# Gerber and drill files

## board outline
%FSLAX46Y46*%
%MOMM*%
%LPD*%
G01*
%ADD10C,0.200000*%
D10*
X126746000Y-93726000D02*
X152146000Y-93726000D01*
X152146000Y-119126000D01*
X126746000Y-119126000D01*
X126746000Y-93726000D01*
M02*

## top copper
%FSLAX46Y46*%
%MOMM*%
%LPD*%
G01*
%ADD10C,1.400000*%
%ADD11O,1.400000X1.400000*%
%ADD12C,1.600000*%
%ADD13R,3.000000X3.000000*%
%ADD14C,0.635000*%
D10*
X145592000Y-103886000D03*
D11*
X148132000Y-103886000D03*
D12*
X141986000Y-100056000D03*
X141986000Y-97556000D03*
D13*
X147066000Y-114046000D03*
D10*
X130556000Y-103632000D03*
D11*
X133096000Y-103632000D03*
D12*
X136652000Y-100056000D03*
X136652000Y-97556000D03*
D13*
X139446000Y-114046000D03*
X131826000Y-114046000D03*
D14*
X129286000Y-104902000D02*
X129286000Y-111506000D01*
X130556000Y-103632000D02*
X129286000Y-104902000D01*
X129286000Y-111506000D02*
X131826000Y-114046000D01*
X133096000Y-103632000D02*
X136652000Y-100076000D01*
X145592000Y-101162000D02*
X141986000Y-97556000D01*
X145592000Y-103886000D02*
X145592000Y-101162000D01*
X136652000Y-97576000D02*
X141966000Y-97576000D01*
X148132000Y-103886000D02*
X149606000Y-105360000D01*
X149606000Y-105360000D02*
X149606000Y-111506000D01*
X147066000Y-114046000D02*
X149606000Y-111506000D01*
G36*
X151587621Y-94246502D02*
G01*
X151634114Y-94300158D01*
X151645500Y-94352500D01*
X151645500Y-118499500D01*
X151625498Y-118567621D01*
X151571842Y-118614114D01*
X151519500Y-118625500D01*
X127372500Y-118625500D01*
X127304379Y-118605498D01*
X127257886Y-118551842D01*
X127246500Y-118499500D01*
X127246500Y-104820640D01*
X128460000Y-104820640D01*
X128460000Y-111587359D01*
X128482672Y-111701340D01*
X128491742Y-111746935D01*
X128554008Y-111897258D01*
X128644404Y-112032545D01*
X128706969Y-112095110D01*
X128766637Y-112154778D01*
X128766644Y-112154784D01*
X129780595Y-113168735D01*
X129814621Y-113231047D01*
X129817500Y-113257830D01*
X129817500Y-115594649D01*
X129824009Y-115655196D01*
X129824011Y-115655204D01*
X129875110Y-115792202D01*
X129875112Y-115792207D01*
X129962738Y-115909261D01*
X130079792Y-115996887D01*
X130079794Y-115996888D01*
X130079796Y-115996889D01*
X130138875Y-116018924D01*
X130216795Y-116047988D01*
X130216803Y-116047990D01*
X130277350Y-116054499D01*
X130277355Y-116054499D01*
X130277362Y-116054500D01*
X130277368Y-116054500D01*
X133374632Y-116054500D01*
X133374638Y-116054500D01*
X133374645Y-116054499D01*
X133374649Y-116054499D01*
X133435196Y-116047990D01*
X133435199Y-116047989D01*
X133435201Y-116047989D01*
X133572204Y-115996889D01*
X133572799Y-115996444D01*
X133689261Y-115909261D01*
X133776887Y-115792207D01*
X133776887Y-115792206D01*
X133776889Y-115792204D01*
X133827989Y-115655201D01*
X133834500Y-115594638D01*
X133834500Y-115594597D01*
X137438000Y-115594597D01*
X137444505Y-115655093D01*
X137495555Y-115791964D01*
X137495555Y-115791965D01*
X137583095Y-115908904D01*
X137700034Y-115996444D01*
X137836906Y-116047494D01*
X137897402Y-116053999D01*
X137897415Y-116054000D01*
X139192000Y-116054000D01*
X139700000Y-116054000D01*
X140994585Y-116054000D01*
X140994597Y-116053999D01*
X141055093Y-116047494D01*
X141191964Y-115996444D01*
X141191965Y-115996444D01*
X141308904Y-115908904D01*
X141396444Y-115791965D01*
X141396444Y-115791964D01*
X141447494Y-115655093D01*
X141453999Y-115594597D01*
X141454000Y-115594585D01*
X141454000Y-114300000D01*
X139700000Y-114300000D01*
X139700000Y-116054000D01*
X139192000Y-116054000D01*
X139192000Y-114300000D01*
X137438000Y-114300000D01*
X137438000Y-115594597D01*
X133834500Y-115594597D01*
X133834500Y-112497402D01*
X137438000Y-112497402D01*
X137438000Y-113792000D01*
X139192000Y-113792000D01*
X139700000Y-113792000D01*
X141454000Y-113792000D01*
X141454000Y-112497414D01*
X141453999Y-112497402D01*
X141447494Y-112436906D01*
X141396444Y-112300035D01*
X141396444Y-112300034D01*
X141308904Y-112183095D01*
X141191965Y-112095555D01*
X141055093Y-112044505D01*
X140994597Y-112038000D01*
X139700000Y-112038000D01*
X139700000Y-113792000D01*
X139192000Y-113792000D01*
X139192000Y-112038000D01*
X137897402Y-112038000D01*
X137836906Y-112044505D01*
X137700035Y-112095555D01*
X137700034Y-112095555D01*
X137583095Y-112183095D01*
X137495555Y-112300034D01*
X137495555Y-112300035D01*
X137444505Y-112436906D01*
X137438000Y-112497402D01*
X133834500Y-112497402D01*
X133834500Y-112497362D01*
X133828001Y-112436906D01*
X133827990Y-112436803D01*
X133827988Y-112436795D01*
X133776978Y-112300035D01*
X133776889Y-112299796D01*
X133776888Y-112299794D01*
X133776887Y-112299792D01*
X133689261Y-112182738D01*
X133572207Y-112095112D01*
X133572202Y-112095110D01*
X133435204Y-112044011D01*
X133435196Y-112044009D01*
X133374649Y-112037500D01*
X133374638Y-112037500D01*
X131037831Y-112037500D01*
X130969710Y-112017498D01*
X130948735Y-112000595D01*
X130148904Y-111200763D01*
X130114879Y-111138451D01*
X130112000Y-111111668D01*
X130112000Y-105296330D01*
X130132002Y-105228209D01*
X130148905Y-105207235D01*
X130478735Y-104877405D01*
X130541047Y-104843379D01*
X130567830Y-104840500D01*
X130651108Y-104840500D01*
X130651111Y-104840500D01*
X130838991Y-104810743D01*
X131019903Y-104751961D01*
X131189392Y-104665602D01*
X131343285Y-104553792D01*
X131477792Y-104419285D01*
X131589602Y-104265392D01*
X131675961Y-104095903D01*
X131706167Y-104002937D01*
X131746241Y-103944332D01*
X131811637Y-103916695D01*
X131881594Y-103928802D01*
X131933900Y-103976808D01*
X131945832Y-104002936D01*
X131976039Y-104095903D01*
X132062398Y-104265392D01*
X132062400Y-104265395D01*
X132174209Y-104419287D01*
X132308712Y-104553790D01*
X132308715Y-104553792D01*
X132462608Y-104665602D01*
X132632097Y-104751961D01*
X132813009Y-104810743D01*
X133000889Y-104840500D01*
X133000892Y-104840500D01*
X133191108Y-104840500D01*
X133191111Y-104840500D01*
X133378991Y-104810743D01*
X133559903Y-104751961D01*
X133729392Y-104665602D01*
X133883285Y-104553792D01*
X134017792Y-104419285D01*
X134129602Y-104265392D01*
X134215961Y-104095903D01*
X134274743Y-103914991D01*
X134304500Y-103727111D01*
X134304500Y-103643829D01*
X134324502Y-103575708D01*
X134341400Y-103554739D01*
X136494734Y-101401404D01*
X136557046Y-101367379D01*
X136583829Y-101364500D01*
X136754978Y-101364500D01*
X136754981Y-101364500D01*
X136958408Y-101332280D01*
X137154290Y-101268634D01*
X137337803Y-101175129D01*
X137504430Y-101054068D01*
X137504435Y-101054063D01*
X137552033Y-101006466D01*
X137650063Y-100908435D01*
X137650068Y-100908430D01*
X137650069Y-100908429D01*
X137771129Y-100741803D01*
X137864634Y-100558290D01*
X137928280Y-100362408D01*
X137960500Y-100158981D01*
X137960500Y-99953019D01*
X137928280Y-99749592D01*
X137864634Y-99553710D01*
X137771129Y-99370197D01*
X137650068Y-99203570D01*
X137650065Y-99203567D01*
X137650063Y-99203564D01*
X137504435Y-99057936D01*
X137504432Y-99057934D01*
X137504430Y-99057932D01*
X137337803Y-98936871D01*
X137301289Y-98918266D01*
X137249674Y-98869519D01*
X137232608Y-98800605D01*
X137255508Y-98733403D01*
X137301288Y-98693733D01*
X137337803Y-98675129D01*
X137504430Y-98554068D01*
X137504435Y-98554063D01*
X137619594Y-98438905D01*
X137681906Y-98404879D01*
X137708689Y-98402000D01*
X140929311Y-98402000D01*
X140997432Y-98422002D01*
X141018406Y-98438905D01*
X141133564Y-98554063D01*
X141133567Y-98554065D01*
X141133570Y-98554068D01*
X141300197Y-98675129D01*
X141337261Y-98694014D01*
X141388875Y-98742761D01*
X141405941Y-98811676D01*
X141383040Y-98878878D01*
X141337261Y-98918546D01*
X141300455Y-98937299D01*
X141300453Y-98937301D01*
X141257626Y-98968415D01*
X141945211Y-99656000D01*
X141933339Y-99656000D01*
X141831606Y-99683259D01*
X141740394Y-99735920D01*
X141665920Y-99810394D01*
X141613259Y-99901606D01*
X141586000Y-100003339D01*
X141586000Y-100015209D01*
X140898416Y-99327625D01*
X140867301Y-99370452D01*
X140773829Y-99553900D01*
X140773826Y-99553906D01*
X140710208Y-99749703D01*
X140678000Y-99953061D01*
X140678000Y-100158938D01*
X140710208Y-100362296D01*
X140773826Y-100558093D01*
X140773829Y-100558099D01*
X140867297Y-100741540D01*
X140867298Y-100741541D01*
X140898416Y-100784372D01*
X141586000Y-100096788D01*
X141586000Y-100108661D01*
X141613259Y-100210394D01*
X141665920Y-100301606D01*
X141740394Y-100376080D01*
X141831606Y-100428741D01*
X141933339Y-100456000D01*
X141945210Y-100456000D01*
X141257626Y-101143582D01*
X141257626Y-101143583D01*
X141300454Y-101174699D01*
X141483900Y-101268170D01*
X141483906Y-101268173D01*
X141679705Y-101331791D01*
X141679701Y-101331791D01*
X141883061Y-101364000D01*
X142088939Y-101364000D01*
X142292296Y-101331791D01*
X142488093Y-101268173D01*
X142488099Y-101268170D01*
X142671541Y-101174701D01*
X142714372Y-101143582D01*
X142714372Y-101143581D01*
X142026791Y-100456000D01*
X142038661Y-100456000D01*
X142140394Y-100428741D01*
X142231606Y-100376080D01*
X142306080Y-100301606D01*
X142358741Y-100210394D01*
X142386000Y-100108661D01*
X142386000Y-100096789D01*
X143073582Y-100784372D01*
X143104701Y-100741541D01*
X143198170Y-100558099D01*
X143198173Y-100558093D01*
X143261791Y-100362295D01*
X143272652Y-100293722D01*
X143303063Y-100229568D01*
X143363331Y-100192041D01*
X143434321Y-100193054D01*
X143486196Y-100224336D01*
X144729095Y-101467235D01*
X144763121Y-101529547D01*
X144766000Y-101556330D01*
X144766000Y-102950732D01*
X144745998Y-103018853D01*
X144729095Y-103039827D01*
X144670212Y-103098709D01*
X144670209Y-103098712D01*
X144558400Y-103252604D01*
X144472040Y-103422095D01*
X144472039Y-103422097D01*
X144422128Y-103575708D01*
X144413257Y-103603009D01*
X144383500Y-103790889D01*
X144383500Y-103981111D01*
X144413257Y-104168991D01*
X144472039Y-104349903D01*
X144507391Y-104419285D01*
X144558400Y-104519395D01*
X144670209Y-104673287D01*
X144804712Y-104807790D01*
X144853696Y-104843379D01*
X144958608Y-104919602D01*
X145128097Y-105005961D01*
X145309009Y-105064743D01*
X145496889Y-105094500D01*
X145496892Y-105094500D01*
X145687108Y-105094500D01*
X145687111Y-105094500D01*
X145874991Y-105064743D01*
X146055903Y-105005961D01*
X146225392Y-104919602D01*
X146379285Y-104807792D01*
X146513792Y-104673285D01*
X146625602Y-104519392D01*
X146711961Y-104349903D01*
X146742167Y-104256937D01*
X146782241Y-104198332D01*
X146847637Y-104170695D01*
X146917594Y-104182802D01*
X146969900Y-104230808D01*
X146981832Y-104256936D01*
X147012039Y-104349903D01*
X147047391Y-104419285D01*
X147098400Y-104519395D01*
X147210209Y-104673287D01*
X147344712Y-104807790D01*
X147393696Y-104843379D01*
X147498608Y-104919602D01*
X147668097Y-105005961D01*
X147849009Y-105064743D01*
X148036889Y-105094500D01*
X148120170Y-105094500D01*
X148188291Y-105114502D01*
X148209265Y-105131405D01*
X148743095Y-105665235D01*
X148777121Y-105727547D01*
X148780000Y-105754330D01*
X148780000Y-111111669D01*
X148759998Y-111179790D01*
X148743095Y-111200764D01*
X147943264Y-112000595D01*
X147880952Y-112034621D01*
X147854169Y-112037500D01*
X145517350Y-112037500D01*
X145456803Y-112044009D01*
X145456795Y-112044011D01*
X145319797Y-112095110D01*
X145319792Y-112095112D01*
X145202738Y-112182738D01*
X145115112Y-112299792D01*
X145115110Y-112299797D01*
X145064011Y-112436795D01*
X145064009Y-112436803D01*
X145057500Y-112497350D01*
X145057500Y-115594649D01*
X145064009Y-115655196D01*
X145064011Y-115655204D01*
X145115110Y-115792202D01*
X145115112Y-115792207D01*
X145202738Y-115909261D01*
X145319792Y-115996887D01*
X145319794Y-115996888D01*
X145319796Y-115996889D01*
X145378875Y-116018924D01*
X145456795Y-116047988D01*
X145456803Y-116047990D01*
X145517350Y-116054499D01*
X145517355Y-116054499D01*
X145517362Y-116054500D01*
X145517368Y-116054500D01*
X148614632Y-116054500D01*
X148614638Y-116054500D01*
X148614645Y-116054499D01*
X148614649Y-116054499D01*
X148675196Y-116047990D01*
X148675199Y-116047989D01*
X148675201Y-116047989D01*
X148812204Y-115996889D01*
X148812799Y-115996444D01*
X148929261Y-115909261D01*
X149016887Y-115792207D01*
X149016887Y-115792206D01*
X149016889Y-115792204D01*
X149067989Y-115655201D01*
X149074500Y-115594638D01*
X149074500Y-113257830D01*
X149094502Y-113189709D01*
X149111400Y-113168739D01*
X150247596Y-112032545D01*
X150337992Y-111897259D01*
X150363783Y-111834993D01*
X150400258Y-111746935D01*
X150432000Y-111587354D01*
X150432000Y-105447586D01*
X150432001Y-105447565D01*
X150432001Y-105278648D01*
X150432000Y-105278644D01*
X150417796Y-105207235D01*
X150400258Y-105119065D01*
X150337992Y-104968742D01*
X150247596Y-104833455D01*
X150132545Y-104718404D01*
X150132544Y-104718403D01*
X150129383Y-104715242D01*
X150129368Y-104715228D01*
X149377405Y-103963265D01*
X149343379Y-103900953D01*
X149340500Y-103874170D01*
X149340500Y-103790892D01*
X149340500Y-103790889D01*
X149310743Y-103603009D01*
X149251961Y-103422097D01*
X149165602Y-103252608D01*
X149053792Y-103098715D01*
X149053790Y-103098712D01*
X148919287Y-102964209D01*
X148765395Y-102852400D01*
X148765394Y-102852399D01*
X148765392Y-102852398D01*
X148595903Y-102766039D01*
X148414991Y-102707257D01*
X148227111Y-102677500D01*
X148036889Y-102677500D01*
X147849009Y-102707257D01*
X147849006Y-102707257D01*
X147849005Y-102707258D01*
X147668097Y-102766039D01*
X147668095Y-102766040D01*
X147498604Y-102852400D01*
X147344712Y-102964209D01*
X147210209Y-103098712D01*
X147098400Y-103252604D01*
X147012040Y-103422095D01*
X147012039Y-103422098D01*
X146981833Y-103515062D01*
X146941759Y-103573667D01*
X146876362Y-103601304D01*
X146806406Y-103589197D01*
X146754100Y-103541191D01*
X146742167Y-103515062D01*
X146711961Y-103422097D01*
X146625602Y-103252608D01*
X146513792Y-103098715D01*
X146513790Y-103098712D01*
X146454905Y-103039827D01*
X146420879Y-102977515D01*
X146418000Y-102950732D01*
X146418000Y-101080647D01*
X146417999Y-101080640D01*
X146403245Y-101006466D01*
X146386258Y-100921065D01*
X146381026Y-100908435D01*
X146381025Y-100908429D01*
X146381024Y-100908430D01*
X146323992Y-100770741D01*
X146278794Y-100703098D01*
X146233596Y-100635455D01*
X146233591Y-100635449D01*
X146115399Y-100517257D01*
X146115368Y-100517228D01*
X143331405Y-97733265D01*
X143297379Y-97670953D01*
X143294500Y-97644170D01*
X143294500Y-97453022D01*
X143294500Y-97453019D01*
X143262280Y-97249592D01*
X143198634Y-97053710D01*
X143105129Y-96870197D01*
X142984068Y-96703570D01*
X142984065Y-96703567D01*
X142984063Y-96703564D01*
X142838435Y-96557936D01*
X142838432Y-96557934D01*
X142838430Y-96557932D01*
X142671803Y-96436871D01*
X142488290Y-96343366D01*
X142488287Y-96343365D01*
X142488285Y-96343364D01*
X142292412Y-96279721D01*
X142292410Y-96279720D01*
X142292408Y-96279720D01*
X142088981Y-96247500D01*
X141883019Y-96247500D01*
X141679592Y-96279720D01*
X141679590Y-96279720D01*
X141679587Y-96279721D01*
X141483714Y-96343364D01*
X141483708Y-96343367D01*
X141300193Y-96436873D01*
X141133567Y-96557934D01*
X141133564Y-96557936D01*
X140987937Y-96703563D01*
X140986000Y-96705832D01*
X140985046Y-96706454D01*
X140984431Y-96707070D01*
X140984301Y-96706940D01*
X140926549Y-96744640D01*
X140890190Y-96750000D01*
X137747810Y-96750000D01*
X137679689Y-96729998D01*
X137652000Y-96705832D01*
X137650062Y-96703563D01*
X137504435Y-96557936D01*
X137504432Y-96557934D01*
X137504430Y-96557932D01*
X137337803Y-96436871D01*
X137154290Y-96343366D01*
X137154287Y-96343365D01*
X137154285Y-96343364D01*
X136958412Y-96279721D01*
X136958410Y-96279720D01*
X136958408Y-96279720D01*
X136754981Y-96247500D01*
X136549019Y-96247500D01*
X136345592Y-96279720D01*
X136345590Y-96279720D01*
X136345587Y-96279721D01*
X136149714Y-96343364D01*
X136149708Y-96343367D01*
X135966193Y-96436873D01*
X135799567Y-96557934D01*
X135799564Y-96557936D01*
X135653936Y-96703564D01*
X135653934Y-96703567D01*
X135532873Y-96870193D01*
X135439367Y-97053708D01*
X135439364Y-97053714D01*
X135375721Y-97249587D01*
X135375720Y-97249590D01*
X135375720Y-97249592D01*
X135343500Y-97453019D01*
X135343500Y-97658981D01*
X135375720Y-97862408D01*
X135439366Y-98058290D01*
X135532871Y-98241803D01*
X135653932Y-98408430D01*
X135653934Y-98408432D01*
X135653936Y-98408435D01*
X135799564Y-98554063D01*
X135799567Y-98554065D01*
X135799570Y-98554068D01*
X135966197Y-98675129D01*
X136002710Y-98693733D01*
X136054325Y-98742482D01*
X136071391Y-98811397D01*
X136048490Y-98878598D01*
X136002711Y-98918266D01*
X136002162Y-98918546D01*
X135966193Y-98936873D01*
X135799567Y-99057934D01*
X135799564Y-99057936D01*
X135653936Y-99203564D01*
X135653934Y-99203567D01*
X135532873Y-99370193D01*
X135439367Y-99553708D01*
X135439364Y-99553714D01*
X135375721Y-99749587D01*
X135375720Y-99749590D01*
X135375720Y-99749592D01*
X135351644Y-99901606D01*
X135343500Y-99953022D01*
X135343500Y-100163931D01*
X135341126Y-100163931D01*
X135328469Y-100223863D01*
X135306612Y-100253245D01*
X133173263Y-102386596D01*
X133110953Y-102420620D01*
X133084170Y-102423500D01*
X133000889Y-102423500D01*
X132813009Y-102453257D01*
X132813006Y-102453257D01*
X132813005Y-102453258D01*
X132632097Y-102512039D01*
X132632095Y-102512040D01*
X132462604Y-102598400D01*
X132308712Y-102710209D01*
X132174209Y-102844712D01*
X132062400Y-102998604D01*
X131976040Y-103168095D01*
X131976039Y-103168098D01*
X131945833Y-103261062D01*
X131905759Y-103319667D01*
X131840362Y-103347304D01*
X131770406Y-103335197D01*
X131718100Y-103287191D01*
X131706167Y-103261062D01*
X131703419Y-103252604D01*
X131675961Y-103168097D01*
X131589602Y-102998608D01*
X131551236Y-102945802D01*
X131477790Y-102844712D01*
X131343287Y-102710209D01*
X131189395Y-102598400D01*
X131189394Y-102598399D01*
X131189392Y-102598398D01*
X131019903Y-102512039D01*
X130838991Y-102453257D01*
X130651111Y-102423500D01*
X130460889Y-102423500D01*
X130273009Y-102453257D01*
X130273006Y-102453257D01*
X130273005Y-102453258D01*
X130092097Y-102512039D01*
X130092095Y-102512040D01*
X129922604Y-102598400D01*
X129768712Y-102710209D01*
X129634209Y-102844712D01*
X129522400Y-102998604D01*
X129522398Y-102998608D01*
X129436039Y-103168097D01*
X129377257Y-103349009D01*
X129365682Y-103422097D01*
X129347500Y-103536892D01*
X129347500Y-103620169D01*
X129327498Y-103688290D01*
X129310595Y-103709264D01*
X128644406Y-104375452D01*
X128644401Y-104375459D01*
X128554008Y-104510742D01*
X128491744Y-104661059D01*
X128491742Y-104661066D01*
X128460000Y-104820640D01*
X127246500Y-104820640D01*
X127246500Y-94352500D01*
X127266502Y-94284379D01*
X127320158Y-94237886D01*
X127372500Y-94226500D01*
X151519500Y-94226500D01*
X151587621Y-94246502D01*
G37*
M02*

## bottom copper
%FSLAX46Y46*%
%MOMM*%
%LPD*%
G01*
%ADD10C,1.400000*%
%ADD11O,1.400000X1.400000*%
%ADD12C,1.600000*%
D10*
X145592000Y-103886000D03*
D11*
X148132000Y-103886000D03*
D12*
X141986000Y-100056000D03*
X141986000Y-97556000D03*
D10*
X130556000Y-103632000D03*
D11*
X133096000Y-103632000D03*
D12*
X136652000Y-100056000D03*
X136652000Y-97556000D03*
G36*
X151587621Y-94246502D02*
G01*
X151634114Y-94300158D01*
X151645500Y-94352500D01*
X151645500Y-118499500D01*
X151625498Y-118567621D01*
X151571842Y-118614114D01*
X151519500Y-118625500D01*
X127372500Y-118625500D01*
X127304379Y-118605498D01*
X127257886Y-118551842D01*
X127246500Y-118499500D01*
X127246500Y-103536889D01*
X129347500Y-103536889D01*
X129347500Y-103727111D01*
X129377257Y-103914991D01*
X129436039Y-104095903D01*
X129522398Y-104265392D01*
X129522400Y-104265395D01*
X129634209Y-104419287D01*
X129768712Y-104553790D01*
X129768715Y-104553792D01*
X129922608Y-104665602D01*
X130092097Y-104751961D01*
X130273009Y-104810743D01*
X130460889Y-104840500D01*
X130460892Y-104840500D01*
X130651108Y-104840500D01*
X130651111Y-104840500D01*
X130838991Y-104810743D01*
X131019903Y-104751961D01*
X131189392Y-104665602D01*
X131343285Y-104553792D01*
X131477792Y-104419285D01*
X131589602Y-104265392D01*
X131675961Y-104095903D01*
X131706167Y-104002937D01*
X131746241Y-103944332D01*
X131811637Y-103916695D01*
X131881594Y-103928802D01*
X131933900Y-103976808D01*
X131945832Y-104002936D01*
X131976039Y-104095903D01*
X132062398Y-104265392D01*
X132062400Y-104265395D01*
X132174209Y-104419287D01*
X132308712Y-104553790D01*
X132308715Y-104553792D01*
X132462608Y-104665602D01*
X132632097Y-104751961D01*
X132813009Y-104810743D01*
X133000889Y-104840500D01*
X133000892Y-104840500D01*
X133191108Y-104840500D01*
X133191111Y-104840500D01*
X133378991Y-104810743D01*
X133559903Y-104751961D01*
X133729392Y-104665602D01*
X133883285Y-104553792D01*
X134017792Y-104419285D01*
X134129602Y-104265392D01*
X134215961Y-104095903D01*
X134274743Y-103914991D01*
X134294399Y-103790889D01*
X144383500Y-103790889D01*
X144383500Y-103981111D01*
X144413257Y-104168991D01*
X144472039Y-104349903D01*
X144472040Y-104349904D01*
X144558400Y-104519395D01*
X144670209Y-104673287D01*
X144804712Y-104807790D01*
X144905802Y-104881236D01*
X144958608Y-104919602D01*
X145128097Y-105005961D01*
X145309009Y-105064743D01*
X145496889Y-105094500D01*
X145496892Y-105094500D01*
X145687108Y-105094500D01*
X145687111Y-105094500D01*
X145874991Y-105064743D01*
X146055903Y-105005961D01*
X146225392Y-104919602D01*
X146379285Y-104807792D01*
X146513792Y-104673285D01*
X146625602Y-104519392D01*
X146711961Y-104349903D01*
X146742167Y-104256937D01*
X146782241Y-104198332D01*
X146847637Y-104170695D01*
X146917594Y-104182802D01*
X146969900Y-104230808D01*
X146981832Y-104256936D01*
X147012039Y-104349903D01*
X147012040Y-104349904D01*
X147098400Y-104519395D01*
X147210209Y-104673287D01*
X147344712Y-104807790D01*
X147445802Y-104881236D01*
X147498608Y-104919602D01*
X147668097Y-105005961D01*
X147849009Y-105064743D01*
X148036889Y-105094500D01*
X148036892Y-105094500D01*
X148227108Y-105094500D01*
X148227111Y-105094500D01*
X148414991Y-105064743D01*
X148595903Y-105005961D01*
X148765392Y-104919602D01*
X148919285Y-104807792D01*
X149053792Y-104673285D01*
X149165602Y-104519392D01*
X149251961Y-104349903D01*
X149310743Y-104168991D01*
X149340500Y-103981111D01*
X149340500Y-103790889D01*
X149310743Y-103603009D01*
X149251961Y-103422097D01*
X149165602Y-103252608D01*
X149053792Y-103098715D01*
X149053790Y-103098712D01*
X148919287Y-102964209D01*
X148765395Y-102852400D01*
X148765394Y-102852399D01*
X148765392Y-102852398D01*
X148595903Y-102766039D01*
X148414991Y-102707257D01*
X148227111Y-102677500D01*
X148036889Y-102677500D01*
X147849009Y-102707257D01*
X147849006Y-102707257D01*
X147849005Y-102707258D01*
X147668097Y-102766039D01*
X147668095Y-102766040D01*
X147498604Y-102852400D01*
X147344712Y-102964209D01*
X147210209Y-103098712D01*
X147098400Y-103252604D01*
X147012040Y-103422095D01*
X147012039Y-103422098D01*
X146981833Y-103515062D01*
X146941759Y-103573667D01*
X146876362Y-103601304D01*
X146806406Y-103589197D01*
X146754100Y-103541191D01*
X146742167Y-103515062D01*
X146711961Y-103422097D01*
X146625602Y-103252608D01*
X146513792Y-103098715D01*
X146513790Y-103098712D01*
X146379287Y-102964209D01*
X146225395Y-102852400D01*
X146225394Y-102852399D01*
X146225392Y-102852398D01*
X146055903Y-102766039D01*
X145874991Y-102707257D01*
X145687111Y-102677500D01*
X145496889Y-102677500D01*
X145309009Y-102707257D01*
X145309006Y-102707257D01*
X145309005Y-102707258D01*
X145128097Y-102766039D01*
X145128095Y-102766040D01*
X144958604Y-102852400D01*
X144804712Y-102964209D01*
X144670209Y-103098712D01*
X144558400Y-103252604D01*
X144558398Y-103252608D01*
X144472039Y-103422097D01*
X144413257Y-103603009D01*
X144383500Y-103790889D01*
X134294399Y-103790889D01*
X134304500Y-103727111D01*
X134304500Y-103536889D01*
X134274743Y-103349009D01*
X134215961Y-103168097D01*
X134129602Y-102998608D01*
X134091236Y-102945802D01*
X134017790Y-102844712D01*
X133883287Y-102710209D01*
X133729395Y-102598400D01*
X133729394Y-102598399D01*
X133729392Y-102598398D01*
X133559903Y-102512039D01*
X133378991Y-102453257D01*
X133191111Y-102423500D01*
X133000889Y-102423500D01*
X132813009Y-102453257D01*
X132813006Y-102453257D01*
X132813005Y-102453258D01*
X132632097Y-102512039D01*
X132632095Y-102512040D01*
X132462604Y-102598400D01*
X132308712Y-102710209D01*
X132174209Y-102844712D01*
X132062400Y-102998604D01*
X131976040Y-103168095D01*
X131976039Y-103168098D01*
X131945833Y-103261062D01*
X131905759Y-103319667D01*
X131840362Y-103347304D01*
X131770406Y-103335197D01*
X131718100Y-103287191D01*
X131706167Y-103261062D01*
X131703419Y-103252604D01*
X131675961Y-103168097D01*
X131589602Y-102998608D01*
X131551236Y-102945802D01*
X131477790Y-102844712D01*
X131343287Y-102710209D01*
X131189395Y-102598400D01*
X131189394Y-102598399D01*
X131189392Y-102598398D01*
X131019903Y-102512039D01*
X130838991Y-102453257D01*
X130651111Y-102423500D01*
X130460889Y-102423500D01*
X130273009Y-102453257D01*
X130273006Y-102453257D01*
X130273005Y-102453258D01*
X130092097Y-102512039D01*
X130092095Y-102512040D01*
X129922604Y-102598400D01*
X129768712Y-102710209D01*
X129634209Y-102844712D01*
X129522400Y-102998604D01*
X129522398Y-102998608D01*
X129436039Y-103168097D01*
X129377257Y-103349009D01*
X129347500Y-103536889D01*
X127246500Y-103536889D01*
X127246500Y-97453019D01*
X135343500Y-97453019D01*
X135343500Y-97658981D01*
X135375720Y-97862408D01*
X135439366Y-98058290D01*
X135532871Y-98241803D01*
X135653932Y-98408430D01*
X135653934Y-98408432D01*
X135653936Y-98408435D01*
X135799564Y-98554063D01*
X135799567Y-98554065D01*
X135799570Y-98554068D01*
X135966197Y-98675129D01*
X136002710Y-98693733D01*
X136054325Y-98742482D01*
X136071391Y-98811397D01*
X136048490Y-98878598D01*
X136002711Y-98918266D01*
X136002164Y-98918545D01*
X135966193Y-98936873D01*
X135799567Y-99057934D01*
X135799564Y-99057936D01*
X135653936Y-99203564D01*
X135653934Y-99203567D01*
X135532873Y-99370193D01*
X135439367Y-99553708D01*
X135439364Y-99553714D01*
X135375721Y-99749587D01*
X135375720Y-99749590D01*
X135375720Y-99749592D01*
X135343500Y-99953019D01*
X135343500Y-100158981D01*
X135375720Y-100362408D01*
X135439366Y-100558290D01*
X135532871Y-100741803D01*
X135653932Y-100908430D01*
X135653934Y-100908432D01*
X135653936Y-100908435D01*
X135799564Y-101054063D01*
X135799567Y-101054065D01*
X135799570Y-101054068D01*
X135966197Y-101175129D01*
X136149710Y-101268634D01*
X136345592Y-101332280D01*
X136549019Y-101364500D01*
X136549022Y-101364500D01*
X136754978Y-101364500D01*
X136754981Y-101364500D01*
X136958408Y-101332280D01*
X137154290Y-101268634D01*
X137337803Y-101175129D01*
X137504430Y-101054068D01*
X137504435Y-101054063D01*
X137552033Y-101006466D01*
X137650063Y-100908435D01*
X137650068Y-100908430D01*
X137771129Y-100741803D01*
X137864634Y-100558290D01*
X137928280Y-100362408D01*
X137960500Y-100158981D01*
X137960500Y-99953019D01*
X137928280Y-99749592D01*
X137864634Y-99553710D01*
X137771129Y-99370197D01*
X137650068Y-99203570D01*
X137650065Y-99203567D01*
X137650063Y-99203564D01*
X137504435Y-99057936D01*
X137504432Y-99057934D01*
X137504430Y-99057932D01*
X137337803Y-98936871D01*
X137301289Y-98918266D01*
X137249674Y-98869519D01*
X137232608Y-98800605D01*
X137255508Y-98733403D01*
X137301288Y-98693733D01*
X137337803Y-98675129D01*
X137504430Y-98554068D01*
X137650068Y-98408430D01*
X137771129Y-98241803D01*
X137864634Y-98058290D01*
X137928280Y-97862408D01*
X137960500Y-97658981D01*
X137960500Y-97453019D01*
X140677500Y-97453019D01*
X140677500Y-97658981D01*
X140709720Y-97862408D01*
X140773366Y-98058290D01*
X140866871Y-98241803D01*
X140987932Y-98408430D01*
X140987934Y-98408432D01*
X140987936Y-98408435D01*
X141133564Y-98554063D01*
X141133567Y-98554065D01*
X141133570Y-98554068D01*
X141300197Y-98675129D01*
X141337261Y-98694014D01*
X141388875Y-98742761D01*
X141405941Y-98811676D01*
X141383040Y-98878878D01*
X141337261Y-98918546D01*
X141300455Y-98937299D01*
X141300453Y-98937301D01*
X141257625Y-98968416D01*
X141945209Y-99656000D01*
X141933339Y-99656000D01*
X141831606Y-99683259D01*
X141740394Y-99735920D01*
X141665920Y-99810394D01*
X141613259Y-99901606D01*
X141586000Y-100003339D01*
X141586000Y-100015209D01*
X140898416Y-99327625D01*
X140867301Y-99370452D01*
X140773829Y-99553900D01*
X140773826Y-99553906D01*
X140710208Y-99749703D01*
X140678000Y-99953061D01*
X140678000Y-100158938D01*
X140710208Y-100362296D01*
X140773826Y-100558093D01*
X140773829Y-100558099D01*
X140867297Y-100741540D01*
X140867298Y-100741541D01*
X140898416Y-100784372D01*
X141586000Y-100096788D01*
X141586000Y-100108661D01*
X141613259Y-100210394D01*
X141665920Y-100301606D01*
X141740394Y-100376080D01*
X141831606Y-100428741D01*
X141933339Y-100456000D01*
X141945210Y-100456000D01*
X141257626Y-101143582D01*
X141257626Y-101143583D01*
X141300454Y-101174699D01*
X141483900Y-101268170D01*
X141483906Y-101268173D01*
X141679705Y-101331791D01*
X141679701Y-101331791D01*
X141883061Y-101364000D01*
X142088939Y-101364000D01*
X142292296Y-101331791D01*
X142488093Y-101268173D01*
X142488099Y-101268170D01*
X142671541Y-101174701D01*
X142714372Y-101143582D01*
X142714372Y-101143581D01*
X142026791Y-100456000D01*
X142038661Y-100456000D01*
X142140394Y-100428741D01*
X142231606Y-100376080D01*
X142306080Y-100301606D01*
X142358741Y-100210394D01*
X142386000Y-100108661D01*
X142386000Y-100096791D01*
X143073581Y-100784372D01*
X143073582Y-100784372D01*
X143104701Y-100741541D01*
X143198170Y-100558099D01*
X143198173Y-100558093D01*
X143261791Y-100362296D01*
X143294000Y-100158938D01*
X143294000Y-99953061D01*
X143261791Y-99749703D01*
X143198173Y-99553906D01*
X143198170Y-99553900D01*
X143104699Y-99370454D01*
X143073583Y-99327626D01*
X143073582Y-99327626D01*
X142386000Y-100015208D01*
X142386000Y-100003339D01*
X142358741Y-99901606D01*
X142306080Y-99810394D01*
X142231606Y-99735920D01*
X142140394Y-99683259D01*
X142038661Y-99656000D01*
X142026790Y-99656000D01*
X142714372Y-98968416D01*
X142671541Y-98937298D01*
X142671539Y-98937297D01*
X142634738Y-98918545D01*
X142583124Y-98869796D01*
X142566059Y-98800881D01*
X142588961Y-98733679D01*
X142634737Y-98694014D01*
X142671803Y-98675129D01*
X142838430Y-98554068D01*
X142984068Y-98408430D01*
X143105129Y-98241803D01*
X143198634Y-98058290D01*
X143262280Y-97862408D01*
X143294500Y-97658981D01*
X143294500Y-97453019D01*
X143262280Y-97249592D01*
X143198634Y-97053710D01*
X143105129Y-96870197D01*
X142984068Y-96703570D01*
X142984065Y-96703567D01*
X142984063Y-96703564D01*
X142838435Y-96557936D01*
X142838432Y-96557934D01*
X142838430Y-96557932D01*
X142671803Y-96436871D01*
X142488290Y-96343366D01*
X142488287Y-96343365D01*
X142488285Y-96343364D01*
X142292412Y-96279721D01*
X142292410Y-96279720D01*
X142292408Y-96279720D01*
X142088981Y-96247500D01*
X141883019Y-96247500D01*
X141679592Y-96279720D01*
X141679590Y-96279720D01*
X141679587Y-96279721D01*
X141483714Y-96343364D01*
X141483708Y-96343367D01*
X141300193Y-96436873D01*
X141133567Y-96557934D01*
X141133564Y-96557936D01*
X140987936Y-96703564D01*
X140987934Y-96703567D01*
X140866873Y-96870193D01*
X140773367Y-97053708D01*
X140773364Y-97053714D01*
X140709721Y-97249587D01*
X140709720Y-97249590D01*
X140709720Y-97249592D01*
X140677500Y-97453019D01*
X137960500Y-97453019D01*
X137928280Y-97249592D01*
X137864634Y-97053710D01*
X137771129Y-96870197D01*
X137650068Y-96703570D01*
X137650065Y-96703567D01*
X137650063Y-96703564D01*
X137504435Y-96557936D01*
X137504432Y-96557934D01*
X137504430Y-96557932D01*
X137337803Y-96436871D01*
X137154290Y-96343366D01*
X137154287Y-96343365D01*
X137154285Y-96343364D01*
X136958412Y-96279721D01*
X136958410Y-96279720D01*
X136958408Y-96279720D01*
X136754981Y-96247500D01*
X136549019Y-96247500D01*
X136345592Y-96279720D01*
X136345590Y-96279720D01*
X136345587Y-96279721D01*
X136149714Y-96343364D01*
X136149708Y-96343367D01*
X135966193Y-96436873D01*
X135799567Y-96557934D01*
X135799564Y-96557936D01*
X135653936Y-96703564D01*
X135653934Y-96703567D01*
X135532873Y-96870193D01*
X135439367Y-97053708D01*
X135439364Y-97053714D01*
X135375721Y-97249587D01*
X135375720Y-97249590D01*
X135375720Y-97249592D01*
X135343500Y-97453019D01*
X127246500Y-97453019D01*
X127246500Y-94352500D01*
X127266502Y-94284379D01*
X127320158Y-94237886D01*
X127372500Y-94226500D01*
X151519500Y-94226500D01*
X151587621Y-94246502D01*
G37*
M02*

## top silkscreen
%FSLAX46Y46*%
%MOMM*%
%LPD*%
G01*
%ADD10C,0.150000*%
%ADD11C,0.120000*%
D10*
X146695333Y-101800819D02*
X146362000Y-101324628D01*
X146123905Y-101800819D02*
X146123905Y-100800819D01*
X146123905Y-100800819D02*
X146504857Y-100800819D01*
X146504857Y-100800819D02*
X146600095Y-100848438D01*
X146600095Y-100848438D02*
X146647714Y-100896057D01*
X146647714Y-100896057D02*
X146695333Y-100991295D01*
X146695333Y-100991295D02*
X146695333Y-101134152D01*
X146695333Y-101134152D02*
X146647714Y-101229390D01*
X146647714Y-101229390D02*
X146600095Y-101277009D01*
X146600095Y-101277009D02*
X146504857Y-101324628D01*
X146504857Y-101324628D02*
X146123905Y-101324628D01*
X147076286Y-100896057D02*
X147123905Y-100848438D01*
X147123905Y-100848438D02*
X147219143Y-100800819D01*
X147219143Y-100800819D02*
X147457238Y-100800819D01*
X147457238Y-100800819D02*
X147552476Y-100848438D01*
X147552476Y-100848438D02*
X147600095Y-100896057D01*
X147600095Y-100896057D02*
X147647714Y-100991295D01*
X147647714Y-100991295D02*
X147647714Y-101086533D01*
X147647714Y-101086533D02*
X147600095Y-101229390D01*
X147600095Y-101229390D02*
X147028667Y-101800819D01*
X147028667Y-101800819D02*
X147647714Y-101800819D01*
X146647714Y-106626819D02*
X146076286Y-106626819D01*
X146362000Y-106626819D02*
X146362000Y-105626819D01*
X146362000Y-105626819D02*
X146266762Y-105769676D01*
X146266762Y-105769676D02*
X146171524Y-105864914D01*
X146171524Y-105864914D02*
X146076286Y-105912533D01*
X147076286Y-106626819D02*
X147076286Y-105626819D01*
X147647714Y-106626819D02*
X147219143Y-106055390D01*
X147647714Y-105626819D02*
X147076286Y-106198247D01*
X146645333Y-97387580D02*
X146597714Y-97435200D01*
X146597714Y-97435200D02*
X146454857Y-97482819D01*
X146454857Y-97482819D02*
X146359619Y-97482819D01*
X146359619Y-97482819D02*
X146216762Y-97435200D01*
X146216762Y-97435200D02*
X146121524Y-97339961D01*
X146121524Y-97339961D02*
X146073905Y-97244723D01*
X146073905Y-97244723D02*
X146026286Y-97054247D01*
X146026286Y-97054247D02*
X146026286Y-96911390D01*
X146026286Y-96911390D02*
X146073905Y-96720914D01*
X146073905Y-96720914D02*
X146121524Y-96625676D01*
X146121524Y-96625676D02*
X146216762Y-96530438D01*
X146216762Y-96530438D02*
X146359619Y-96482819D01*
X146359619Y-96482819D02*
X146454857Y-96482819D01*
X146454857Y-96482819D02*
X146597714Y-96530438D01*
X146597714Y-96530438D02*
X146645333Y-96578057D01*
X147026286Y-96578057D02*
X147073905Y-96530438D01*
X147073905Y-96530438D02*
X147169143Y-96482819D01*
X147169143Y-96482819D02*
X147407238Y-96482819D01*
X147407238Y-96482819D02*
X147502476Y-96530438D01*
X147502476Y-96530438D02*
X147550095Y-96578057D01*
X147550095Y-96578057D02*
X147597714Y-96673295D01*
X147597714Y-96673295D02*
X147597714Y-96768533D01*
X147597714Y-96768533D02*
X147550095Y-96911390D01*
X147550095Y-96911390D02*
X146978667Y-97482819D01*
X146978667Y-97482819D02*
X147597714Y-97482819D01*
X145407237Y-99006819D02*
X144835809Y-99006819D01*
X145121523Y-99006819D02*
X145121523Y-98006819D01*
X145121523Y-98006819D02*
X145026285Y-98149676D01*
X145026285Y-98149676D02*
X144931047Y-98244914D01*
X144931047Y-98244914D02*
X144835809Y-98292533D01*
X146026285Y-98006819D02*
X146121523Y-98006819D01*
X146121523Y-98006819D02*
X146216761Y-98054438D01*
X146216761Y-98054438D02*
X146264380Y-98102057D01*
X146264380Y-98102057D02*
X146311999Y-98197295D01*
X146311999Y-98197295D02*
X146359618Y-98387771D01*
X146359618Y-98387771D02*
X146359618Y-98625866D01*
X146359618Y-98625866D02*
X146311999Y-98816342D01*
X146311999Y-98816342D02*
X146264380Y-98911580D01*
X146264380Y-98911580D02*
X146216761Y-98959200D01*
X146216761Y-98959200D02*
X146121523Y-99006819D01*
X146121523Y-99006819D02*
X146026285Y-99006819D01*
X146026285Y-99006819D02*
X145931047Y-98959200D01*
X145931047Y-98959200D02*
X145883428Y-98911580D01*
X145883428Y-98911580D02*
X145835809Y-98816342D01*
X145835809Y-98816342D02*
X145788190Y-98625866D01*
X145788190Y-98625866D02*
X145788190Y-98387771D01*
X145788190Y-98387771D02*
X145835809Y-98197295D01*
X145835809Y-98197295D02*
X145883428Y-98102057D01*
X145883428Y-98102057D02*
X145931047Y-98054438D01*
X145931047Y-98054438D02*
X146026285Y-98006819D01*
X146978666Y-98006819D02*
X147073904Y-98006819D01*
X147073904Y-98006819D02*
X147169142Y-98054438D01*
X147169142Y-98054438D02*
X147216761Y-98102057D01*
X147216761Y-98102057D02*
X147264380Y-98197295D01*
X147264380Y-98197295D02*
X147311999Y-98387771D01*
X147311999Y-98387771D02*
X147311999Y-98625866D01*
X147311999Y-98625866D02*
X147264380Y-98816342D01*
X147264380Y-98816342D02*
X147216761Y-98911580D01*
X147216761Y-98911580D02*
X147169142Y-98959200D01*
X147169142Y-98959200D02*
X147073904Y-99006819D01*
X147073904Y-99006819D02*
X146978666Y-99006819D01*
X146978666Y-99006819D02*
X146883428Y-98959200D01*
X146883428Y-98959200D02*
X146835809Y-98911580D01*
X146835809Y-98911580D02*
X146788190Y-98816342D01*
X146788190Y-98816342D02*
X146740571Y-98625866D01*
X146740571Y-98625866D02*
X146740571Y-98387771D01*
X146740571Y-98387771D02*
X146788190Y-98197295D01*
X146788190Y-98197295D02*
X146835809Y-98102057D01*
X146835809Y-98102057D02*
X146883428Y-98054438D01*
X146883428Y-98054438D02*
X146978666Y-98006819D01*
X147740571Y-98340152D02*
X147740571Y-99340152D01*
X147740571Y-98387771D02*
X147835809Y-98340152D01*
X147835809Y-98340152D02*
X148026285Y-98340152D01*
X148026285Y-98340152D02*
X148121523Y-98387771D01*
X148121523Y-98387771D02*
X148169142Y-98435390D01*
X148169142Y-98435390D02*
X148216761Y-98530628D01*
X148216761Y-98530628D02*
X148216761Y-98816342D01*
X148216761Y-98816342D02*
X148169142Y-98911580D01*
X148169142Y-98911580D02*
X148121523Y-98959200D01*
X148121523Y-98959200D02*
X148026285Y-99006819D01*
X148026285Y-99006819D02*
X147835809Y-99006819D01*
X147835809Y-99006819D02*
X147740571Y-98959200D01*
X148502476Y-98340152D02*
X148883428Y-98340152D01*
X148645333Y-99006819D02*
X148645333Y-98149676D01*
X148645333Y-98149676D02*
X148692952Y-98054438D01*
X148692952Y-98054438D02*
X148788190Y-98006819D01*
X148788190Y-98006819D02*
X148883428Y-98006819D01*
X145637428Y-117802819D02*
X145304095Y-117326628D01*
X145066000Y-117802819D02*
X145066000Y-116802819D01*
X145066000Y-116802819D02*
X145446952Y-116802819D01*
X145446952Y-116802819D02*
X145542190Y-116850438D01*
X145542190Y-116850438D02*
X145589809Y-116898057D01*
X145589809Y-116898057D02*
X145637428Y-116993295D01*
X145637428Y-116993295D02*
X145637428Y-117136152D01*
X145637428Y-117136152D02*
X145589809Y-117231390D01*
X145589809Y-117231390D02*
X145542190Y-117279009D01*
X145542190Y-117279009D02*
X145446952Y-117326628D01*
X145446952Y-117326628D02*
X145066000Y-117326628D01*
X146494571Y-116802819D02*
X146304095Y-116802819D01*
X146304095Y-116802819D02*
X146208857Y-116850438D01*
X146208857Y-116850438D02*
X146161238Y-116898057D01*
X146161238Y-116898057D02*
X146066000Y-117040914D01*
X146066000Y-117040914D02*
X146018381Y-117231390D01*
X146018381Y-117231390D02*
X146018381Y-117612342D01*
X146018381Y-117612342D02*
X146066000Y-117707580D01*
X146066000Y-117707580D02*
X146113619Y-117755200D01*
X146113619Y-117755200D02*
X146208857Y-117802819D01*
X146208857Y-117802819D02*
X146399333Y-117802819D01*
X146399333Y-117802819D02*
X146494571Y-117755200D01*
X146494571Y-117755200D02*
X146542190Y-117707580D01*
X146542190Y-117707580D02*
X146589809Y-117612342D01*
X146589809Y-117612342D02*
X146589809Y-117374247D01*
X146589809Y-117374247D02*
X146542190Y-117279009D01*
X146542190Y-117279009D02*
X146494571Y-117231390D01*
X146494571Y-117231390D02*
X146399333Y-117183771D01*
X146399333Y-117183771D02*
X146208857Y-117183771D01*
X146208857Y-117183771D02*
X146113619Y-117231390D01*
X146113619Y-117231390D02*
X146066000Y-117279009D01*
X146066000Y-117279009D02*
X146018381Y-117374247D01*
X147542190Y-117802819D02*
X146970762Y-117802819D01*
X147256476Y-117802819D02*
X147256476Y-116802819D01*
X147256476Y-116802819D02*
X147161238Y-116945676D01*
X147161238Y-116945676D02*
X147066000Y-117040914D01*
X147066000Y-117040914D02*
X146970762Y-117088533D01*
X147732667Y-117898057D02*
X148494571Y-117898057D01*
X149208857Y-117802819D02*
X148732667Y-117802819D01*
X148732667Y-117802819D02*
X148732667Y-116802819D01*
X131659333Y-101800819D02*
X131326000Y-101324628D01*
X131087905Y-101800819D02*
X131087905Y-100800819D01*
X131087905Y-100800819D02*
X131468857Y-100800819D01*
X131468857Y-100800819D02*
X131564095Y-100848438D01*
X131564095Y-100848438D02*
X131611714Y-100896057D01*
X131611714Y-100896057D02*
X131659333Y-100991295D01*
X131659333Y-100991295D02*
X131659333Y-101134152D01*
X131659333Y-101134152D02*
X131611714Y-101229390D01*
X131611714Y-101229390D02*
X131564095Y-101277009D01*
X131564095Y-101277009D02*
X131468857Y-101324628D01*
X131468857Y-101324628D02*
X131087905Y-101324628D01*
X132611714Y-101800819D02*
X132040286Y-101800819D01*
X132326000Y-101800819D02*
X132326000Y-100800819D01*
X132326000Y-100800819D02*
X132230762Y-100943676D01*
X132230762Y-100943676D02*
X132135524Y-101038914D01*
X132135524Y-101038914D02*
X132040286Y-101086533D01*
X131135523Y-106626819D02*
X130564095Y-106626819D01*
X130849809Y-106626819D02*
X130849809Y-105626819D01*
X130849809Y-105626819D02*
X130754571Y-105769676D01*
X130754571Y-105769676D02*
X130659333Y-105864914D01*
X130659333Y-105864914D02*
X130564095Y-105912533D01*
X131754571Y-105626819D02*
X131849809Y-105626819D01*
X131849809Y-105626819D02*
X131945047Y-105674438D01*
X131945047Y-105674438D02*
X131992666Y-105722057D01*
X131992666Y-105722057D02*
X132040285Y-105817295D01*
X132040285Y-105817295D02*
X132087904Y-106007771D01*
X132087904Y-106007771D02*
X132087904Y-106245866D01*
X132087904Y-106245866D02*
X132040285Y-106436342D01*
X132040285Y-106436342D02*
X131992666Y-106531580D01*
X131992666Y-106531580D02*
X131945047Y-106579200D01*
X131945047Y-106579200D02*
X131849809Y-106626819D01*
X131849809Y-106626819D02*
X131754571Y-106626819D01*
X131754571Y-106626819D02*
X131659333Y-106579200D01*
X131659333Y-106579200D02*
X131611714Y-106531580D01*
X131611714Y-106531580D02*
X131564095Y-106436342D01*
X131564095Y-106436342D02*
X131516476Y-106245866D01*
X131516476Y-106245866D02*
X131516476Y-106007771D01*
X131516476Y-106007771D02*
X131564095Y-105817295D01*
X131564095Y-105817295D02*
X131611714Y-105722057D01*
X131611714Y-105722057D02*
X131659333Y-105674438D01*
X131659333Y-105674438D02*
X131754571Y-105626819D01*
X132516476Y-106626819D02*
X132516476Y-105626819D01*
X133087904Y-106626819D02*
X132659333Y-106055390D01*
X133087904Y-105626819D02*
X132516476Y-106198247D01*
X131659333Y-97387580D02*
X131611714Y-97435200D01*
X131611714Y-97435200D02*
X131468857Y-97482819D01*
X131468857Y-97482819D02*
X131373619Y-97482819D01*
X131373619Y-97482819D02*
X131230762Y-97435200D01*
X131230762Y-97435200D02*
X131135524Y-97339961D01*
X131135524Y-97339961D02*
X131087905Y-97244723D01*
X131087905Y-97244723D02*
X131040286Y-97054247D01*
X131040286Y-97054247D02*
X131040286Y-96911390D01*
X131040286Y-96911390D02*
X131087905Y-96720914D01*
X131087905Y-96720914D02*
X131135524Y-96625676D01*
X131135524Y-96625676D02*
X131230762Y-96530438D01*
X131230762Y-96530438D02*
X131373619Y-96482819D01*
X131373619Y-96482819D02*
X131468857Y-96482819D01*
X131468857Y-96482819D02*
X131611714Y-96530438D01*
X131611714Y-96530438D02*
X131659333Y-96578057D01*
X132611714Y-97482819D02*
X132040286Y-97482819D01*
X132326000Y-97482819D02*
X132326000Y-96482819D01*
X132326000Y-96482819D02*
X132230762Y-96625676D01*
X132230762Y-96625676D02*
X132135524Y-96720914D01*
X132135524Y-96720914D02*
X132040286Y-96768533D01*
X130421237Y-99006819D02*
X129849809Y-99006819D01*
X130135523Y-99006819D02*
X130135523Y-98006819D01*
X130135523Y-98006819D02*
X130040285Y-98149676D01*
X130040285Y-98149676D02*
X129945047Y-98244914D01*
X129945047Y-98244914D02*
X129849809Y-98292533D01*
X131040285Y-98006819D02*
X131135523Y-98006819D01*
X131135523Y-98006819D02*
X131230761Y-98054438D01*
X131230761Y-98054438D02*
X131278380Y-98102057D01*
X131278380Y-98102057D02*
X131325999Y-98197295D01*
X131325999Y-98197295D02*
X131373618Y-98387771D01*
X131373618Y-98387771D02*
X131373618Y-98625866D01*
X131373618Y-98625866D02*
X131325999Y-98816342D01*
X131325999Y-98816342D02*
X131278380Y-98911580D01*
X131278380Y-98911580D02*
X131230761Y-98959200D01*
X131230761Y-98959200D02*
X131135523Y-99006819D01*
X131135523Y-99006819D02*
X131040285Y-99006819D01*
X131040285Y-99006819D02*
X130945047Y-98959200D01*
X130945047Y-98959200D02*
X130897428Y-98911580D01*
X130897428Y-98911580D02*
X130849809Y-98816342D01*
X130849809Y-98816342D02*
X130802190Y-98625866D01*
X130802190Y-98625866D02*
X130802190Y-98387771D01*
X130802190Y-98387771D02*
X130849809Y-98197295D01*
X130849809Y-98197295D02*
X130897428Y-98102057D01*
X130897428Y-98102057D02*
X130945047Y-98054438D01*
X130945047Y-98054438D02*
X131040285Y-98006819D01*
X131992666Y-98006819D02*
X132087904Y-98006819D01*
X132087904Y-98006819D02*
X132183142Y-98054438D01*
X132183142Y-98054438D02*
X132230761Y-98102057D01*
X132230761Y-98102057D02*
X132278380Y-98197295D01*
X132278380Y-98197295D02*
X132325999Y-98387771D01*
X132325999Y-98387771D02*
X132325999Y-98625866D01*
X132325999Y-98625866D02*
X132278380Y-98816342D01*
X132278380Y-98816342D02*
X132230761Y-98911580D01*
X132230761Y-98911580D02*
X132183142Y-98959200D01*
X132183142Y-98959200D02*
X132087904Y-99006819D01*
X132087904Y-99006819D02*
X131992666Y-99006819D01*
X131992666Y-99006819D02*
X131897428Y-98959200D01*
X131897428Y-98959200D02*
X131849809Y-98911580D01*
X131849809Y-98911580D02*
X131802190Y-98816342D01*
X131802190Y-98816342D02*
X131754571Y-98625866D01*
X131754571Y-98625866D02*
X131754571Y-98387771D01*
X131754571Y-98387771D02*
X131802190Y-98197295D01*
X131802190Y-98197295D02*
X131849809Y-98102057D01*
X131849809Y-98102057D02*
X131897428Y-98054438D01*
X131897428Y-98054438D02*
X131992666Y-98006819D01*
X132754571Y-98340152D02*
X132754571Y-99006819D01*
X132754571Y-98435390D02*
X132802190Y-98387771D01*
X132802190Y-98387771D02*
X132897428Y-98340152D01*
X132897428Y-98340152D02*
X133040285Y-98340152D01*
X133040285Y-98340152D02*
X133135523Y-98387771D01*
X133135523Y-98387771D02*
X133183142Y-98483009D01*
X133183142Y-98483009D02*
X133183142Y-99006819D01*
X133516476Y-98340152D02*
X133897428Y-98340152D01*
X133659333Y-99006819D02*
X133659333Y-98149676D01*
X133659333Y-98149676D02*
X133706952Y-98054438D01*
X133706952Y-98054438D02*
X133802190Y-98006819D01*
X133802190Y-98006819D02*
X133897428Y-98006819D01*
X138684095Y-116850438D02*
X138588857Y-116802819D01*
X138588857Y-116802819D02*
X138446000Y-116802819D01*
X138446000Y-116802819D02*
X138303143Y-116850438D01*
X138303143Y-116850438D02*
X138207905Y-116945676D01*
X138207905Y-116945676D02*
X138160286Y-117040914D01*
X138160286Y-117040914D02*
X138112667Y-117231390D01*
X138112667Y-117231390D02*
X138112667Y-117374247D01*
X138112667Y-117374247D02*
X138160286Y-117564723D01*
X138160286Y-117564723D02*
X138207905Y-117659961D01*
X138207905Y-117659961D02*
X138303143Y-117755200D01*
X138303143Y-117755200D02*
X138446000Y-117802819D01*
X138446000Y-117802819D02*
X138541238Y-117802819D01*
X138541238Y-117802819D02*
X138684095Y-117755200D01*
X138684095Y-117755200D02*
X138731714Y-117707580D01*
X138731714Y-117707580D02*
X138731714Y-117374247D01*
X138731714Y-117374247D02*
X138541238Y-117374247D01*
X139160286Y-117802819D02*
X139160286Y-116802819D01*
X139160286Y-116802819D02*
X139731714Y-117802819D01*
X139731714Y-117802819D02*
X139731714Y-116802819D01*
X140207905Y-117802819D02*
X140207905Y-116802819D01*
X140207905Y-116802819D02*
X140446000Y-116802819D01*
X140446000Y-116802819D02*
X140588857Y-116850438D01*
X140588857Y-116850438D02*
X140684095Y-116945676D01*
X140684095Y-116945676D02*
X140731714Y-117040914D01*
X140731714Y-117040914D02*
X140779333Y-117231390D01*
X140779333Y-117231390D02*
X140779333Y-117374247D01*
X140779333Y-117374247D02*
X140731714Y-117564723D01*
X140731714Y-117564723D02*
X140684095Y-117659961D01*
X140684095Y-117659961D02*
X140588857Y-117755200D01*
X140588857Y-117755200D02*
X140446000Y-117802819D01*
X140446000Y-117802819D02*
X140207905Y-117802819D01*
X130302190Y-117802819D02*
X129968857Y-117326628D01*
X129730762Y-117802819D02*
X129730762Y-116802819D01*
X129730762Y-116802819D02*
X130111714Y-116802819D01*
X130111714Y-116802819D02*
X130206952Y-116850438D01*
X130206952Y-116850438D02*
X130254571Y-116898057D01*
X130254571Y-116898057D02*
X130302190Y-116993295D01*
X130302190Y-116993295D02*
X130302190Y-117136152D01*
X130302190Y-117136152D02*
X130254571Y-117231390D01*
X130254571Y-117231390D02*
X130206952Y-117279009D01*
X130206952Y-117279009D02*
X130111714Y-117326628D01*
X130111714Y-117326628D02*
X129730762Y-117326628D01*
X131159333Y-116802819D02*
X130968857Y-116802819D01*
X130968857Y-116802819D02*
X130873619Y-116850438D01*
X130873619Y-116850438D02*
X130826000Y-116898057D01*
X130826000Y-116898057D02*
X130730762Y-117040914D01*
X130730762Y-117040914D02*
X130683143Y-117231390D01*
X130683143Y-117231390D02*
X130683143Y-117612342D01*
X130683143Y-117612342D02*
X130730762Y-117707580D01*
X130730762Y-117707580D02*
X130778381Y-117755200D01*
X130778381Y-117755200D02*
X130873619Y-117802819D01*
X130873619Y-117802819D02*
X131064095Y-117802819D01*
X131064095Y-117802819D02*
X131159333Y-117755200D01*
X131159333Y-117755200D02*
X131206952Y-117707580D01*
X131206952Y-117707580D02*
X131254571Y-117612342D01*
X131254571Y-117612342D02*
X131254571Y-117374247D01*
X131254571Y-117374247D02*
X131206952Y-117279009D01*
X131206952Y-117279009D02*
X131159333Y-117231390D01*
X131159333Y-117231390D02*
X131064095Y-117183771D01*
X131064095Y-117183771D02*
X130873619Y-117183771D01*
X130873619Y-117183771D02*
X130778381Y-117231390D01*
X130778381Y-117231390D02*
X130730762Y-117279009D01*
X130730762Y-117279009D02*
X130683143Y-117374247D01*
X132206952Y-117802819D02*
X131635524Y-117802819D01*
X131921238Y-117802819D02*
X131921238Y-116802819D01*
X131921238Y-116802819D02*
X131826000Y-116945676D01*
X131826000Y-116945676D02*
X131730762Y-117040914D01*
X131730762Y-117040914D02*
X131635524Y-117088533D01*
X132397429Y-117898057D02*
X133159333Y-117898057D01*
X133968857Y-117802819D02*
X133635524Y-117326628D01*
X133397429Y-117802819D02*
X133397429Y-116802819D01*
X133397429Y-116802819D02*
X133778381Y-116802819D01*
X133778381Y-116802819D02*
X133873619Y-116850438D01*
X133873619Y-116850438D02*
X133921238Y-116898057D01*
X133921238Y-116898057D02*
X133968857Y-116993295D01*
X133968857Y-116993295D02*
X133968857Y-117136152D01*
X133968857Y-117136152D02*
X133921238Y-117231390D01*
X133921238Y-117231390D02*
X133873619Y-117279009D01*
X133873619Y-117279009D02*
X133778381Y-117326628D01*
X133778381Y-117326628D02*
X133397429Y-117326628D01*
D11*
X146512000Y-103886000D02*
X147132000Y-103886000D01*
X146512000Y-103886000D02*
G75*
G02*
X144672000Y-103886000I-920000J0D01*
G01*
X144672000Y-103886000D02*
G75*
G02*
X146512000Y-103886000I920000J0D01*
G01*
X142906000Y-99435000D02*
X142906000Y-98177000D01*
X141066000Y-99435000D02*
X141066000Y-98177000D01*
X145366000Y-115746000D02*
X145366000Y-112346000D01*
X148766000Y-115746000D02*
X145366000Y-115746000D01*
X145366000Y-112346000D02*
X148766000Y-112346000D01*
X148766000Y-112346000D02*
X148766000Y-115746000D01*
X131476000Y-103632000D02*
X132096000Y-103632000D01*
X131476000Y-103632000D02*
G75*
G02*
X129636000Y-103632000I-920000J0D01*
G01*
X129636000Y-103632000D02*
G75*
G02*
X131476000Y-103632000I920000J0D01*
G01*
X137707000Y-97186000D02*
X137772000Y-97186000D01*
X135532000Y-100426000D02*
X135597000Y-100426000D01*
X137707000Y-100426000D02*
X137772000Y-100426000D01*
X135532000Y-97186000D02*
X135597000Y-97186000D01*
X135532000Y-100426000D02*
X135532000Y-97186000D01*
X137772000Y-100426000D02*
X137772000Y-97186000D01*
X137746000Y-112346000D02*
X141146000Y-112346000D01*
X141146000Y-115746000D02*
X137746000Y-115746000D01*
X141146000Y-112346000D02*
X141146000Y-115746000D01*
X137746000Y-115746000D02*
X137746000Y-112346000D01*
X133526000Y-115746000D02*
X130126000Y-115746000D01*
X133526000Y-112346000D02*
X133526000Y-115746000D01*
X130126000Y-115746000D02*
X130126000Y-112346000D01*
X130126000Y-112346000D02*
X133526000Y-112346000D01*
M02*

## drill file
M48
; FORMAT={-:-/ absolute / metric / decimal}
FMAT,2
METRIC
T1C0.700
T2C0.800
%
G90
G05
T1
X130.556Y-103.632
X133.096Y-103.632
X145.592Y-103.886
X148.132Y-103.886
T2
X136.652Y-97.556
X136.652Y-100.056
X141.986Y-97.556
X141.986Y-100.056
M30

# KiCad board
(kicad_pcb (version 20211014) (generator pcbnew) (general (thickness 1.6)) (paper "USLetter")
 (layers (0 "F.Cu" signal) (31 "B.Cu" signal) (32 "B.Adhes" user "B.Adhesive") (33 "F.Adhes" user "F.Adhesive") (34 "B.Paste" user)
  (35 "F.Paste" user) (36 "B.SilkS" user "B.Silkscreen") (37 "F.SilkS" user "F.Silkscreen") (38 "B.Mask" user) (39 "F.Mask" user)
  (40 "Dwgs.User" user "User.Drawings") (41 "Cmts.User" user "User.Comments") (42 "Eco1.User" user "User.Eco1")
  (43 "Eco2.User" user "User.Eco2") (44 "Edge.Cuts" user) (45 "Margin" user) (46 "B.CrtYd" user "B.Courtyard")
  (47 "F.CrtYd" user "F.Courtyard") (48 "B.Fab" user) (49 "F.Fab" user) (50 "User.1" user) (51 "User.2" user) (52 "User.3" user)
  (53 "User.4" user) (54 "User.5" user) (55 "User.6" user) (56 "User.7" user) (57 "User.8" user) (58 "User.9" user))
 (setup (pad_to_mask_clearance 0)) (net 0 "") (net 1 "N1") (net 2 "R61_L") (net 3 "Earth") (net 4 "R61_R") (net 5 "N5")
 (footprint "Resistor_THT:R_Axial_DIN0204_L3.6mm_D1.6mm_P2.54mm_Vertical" (layer "F.Cu") (at 145.592 103.886)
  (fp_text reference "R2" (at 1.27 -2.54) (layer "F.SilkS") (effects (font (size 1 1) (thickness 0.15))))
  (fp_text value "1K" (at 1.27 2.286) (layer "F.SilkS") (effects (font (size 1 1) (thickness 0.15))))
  (fp_line (start 0.92 0) (end 1.54 0) (layer "F.SilkS") (width 0.12))
  (fp_circle (center 0 0) (end 0.92 0) (layer "F.SilkS") (width 0.12) (fill none))
  (pad "1" thru_hole circle (at 0 0) (size 1.4 1.4) (drill 0.7) (layers *.Cu *.Mask) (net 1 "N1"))
  (pad "2" thru_hole oval (at 2.54 0) (size 1.4 1.4) (drill 0.7) (layers *.Cu *.Mask) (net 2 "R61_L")))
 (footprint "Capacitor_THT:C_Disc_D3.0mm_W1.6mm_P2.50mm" (layer "F.Cu") (at 141.986 100.056 90)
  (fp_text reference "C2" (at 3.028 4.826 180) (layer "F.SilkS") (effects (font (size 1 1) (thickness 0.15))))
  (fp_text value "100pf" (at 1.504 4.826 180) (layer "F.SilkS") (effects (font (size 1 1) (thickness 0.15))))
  (fp_line (start 0.621 0.92) (end 1.879 0.92) (layer "F.SilkS") (width 0.12))
  (fp_line (start 0.621 -0.92) (end 1.879 -0.92) (layer "F.SilkS") (width 0.12))
  (pad "1" thru_hole circle (at 0 0 90) (size 1.6 1.6) (drill 0.8) (layers *.Cu *.Mask) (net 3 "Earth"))
  (pad "2" thru_hole circle (at 2.5 0 90) (size 1.6 1.6) (drill 0.8) (layers *.Cu *.Mask) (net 1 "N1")))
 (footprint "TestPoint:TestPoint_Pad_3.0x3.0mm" (layer "F.Cu") (at 147.066 114.046)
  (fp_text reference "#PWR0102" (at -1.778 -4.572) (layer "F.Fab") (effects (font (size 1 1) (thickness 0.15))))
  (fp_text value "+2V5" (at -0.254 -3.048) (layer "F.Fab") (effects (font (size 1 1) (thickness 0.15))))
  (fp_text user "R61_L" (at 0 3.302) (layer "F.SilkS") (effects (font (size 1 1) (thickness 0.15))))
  (fp_line (start -1.7 1.7) (end -1.7 -1.7) (layer "F.SilkS") (width 0.12))
  (fp_line (start 1.7 1.7) (end -1.7 1.7) (layer "F.SilkS") (width 0.12))
  (fp_line (start -1.7 -1.7) (end 1.7 -1.7) (layer "F.SilkS") (width 0.12))
  (fp_line (start 1.7 -1.7) (end 1.7 1.7) (layer "F.SilkS") (width 0.12))
  (pad "1" smd rect (at 0 0) (size 3 3) (layers "F.Cu" "F.Paste" "F.Mask") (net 2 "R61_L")))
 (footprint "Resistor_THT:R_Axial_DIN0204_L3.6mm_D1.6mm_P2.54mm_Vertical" (layer "F.Cu") (at 130.556 103.632)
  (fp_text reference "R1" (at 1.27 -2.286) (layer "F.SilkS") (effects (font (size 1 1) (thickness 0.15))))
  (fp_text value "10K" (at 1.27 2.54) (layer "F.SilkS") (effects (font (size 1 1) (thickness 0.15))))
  (fp_line (start 0.92 0) (end 1.54 0) (layer "F.SilkS") (width 0.12))
  (fp_circle (center 0 0) (end 0.92 0) (layer "F.SilkS") (width 0.12) (fill none))
  (pad "1" thru_hole circle (at 0 0) (size 1.4 1.4) (drill 0.7) (layers *.Cu *.Mask) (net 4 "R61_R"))
  (pad "2" thru_hole oval (at 2.54 0) (size 1.4 1.4) (drill 0.7) (layers *.Cu *.Mask) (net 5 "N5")))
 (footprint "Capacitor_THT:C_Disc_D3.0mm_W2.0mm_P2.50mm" (layer "F.Cu") (at 136.652 100.056 90)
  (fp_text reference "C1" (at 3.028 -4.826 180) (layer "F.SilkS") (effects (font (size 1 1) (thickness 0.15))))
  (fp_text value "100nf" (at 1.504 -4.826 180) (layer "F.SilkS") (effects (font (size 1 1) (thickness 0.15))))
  (fp_line (start 2.87 1.055) (end 2.87 1.12) (layer "F.SilkS") (width 0.12))
  (fp_line (start -0.37 -1.12) (end -0.37 -1.055) (layer "F.SilkS") (width 0.12))
  (fp_line (start -0.37 1.055) (end -0.37 1.12) (layer "F.SilkS") (width 0.12))
  (fp_line (start 2.87 -1.12) (end 2.87 -1.055) (layer "F.SilkS") (width 0.12))
  (fp_line (start -0.37 -1.12) (end 2.87 -1.12) (layer "F.SilkS") (width 0.12))
  (fp_line (start -0.37 1.12) (end 2.87 1.12) (layer "F.SilkS") (width 0.12))
  (pad "1" thru_hole circle (at 0 0 90) (size 1.6 1.6) (drill 0.8) (layers *.Cu *.Mask) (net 5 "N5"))
  (pad "2" thru_hole circle (at 2.5 0 90) (size 1.6 1.6) (drill 0.8) (layers *.Cu *.Mask) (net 1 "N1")))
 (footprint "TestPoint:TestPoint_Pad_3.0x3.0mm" (layer "F.Cu") (at 139.446 114.046)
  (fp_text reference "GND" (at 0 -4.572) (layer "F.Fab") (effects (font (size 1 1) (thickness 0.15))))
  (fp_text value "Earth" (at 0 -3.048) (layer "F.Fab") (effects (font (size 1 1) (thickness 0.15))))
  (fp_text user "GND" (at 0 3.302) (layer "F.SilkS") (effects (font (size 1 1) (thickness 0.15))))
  (fp_line (start -1.7 -1.7) (end 1.7 -1.7) (layer "F.SilkS") (width 0.12))
  (fp_line (start 1.7 1.7) (end -1.7 1.7) (layer "F.SilkS") (width 0.12))
  (fp_line (start 1.7 -1.7) (end 1.7 1.7) (layer "F.SilkS") (width 0.12))
  (fp_line (start -1.7 1.7) (end -1.7 -1.7) (layer "F.SilkS") (width 0.12))
  (pad "1" smd rect (at 0 0) (size 3 3) (layers "F.Cu" "F.Paste" "F.Mask") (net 3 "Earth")))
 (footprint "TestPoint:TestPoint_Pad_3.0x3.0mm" (layer "F.Cu") (at 131.826 114.046)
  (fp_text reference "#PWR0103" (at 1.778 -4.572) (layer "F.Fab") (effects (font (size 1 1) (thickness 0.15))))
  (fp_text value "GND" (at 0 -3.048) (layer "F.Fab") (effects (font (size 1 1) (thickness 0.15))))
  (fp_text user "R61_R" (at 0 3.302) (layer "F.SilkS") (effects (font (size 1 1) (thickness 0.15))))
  (fp_line (start 1.7 1.7) (end -1.7 1.7) (layer "F.SilkS") (width 0.12))
  (fp_line (start 1.7 -1.7) (end 1.7 1.7) (layer "F.SilkS") (width 0.12))
  (fp_line (start -1.7 1.7) (end -1.7 -1.7) (layer "F.SilkS") (width 0.12))
  (fp_line (start -1.7 -1.7) (end 1.7 -1.7) (layer "F.SilkS") (width 0.12))
  (pad "1" smd rect (at 0 0) (size 3 3) (layers "F.Cu" "F.Paste" "F.Mask") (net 4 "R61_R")))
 (gr_rect (start 126.746 93.726) (end 152.146 119.126) (layer "Edge.Cuts") (width 0.2) (fill none))
 (segment (start 129.286 104.902) (end 129.286 111.506) (width 0.635) (layer "F.Cu") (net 4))
 (segment (start 130.556 103.632) (end 129.286 104.902) (width 0.635) (layer "F.Cu") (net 4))
 (segment (start 129.286 111.506) (end 131.826 114.046) (width 0.635) (layer "F.Cu") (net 4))
 (segment (start 133.096 103.632) (end 136.652 100.076) (width 0.635) (layer "F.Cu") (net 5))
 (segment (start 145.592 101.162) (end 141.986 97.556) (width 0.635) (layer "F.Cu") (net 1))
 (segment (start 145.592 103.886) (end 145.592 101.162) (width 0.635) (layer "F.Cu") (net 1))
 (segment (start 136.652 97.576) (end 141.966 97.576) (width 0.635) (layer "F.Cu") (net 1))
 (segment (start 148.132 103.886) (end 149.606 105.36) (width 0.635) (layer "F.Cu") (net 2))
 (segment (start 149.606 105.36) (end 149.606 111.506) (width 0.635) (layer "F.Cu") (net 2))
 (segment (start 147.066 114.046) (end 149.606 111.506) (width 0.635) (layer "F.Cu") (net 2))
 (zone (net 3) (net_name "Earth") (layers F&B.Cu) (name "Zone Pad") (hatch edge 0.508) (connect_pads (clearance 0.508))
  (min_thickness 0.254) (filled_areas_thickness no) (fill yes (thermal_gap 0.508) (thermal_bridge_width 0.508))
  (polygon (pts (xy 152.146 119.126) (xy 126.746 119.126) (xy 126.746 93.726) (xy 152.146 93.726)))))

